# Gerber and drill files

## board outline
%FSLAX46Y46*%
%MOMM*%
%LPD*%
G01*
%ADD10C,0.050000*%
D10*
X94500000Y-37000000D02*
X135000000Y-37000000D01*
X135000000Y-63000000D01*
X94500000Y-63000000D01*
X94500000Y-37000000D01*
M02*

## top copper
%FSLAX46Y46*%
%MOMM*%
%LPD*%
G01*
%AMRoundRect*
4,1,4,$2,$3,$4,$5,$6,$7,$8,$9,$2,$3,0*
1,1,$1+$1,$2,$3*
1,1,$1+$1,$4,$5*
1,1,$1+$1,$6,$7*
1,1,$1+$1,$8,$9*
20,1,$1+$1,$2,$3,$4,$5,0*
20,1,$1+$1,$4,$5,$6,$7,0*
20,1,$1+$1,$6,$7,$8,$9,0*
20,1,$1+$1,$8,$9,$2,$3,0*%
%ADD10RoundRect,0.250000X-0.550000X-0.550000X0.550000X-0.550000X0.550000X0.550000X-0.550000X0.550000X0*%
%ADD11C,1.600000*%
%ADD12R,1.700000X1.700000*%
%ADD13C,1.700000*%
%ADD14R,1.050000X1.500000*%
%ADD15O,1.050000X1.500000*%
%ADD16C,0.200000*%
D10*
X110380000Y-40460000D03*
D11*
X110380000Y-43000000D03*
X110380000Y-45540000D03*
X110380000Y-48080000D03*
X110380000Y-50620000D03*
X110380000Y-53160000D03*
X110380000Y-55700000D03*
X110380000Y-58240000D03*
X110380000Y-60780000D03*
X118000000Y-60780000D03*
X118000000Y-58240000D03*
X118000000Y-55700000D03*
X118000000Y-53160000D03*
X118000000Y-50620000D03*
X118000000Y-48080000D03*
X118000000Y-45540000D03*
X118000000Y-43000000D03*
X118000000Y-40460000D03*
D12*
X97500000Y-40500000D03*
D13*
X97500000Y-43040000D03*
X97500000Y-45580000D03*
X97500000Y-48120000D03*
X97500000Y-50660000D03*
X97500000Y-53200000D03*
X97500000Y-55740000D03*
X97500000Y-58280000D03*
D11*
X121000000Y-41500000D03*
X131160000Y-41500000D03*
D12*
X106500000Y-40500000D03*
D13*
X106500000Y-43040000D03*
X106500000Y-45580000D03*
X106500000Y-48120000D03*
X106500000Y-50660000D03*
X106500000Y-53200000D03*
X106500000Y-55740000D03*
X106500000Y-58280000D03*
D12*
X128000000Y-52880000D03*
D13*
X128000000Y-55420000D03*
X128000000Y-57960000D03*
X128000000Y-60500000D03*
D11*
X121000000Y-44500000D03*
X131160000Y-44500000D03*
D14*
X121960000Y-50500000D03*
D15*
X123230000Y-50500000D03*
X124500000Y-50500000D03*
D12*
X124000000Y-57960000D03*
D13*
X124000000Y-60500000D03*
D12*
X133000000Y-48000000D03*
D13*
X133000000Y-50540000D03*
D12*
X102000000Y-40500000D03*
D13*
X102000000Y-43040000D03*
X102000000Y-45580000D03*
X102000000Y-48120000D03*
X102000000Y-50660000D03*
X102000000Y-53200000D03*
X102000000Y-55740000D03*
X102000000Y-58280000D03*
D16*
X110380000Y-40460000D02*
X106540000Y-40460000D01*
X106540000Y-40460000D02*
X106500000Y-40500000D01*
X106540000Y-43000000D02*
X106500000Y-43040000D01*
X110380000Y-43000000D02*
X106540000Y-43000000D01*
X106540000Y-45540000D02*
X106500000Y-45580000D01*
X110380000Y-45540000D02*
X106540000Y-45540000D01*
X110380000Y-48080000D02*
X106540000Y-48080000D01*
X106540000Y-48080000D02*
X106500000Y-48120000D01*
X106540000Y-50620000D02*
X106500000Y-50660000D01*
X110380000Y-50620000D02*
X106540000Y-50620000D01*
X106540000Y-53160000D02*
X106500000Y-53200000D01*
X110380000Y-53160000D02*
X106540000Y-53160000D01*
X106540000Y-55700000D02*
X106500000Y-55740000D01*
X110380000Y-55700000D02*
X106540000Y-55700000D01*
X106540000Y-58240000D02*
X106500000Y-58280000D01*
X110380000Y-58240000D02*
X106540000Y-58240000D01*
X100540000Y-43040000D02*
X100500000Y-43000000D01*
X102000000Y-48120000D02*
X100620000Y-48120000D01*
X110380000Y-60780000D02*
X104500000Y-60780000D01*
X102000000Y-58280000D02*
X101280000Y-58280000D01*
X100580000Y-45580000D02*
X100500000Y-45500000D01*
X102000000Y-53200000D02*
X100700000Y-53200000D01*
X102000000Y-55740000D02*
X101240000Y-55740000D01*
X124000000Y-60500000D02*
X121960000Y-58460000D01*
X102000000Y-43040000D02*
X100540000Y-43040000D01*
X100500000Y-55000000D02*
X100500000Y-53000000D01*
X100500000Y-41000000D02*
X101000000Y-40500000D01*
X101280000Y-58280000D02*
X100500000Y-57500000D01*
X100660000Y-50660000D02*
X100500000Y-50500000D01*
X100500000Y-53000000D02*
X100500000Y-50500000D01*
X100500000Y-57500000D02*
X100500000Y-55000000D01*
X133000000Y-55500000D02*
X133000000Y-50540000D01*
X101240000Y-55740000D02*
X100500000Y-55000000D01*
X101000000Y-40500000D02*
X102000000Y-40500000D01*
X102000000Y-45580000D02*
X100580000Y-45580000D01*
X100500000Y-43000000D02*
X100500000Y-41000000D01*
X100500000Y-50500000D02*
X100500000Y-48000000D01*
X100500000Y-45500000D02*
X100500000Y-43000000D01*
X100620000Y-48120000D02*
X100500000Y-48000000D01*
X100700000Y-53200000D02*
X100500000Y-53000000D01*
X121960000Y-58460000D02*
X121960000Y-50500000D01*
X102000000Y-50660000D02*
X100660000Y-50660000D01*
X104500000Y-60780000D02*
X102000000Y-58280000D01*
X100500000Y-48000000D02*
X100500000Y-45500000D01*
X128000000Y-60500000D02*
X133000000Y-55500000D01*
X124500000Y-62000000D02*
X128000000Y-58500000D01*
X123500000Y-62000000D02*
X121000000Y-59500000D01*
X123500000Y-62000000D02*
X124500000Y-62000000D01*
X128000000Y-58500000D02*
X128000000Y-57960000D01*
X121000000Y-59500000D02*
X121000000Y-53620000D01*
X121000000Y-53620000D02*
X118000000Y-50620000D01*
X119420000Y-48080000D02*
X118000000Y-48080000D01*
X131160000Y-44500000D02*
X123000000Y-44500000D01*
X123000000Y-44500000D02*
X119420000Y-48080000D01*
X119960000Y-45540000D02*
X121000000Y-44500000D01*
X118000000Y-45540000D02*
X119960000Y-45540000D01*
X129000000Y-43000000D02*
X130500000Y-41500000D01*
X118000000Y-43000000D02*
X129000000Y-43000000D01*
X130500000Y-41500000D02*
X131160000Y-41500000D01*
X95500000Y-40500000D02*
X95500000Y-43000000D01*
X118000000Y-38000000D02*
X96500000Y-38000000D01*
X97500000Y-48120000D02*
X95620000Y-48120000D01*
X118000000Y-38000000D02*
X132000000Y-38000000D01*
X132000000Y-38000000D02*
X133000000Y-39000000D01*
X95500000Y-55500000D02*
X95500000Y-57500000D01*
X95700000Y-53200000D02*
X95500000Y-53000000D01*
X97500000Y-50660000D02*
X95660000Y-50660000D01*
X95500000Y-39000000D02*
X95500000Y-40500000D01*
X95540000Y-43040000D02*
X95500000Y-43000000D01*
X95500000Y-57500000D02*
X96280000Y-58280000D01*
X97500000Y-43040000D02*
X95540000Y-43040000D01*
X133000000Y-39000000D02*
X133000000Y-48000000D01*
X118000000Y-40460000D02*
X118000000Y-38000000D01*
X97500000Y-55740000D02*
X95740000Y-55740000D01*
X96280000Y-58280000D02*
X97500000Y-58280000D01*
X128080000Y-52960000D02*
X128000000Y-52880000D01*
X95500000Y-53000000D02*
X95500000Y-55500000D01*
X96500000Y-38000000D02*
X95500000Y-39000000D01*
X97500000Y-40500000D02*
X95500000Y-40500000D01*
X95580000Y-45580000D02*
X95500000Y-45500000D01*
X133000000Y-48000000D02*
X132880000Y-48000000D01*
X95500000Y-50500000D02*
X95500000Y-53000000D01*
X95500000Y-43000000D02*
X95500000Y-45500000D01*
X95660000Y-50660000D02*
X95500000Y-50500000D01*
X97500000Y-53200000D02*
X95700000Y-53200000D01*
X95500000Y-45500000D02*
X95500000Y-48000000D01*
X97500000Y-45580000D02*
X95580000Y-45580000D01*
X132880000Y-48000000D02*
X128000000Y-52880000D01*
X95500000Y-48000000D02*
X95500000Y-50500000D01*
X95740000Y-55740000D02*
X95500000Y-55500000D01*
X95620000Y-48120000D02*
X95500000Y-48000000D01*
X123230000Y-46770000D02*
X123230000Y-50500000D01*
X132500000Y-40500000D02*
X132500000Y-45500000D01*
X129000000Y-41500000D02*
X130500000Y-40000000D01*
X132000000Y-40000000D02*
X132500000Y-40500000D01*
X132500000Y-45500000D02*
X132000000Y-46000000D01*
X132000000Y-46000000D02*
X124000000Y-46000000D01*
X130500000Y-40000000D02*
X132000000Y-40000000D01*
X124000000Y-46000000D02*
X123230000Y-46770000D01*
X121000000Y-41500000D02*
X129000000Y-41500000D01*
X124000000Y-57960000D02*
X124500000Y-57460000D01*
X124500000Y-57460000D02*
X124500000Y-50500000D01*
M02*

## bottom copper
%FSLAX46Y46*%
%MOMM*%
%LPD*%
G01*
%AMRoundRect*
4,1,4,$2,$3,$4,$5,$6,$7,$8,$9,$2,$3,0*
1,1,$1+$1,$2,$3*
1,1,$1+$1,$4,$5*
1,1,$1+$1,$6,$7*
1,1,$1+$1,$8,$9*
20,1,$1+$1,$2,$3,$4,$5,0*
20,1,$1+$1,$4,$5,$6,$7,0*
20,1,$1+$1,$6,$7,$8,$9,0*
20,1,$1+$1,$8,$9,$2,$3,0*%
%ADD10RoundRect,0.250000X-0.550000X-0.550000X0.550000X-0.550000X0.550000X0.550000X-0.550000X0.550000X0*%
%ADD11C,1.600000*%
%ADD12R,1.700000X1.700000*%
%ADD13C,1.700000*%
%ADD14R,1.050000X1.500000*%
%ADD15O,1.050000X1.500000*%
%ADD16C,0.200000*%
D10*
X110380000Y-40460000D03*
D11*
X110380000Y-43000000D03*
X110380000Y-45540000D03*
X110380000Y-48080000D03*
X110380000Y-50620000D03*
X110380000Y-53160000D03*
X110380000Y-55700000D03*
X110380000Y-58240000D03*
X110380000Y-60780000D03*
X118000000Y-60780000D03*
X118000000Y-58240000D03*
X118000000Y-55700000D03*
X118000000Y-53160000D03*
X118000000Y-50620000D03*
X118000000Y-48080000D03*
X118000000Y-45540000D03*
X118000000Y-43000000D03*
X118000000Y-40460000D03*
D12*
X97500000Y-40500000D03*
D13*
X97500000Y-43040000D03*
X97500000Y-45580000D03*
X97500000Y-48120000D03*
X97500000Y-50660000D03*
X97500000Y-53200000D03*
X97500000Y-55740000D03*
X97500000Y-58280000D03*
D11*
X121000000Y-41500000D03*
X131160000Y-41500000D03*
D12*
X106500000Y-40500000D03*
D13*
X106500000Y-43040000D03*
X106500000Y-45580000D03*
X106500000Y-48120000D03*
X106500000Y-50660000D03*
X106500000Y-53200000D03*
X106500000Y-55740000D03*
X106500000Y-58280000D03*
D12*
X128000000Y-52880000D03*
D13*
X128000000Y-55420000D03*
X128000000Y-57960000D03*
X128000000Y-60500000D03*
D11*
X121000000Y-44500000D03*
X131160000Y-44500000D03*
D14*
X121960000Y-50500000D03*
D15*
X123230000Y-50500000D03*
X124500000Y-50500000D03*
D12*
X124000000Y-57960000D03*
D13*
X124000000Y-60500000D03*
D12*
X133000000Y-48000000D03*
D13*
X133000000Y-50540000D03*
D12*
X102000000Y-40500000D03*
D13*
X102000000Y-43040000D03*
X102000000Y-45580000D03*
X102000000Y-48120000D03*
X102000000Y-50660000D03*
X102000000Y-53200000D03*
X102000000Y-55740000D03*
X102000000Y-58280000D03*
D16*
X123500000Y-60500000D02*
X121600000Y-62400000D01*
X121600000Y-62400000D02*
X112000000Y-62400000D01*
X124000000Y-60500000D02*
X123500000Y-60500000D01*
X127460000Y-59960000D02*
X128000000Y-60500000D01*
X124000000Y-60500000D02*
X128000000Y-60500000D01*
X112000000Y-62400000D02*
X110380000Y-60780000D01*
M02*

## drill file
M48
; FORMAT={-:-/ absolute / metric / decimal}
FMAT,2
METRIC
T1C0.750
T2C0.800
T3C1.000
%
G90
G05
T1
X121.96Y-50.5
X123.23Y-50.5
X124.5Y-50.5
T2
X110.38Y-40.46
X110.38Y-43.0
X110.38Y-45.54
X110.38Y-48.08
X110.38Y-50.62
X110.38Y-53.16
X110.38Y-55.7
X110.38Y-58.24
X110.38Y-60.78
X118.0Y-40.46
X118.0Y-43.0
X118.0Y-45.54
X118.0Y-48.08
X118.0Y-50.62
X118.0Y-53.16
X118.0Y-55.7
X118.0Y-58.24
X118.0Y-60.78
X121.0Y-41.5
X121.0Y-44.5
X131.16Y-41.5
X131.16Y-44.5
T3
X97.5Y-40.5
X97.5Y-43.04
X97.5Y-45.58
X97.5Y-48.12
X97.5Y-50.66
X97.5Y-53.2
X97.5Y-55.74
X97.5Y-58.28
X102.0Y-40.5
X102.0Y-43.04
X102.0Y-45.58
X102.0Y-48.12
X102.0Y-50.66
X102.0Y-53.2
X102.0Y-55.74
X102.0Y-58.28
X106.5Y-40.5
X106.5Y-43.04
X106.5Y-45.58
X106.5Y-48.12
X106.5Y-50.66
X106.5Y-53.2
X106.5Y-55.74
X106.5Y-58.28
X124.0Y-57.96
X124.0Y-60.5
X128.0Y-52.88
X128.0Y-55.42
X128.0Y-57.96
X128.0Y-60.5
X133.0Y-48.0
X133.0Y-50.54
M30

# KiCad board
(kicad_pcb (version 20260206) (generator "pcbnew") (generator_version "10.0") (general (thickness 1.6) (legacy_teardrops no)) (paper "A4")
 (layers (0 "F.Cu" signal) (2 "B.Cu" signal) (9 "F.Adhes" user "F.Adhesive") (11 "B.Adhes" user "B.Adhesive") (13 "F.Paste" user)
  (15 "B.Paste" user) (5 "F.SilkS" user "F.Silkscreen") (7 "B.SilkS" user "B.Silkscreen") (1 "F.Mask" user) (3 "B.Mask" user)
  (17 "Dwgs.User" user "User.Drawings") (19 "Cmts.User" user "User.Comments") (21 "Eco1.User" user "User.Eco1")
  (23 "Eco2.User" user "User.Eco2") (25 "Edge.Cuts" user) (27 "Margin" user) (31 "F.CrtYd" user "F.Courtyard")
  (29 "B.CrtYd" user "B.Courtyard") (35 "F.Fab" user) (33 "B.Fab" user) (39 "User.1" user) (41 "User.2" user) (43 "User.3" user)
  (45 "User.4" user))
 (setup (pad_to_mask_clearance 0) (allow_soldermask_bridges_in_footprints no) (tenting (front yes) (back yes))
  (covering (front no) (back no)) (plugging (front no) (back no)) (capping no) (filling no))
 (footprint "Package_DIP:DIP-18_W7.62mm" (layer "F.Cu") (at 110.38 40.46)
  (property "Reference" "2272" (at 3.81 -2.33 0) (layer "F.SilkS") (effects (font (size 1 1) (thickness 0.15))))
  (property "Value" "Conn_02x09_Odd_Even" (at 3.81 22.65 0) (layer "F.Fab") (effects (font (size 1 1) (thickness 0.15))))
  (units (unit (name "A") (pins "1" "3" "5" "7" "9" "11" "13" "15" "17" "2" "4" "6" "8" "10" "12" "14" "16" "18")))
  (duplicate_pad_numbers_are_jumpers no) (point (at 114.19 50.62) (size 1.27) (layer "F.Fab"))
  (pad "1" thru_hole roundrect (at 0 0) (size 1.6 1.6) (drill 0.8) (layers "*.Cu" "*.Mask") (remove_unused_layers no)
   (roundrect_rratio 0.15625) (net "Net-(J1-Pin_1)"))
  (pad "2" thru_hole circle (at 0 2.54) (size 1.6 1.6) (drill 0.8) (layers "*.Cu" "*.Mask") (remove_unused_layers no) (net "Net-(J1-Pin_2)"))
  (pad "3" thru_hole circle (at 0 5.08) (size 1.6 1.6) (drill 0.8) (layers "*.Cu" "*.Mask") (remove_unused_layers no) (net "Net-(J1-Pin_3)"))
  (pad "4" thru_hole circle (at 0 7.62) (size 1.6 1.6) (drill 0.8) (layers "*.Cu" "*.Mask") (remove_unused_layers no) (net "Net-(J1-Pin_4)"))
  (pad "5" thru_hole circle (at 0 10.16) (size 1.6 1.6) (drill 0.8) (layers "*.Cu" "*.Mask") (remove_unused_layers no)
   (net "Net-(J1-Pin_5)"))
  (pad "6" thru_hole circle (at 0 12.7) (size 1.6 1.6) (drill 0.8) (layers "*.Cu" "*.Mask") (remove_unused_layers no) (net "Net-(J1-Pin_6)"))
  (pad "7" thru_hole circle (at 0 15.24) (size 1.6 1.6) (drill 0.8) (layers "*.Cu" "*.Mask") (remove_unused_layers no)
   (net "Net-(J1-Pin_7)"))
  (pad "8" thru_hole circle (at 0 17.78) (size 1.6 1.6) (drill 0.8) (layers "*.Cu" "*.Mask") (remove_unused_layers no)
   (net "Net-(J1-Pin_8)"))
  (pad "9" thru_hole circle (at 0 20.32) (size 1.6 1.6) (drill 0.8) (layers "*.Cu" "*.Mask") (remove_unused_layers no) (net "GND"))
  (pad "10" thru_hole circle (at 7.62 20.32) (size 1.6 1.6) (drill 0.8) (layers "*.Cu" "*.Mask") (remove_unused_layers no)
   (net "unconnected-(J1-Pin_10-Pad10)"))
  (pad "11" thru_hole circle (at 7.62 17.78) (size 1.6 1.6) (drill 0.8) (layers "*.Cu" "*.Mask") (remove_unused_layers no)
   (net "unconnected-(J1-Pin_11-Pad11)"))
  (pad "12" thru_hole circle (at 7.62 15.24) (size 1.6 1.6) (drill 0.8) (layers "*.Cu" "*.Mask") (remove_unused_layers no)
   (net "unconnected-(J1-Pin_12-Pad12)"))
  (pad "13" thru_hole circle (at 7.62 12.7) (size 1.6 1.6) (drill 0.8) (layers "*.Cu" "*.Mask") (remove_unused_layers no)
   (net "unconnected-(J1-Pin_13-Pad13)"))
  (pad "14" thru_hole circle (at 7.62 10.16) (size 1.6 1.6) (drill 0.8) (layers "*.Cu" "*.Mask") (remove_unused_layers no)
   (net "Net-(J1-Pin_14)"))
  (pad "15" thru_hole circle (at 7.62 7.62) (size 1.6 1.6) (drill 0.8) (layers "*.Cu" "*.Mask") (remove_unused_layers no)
   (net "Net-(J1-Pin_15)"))
  (pad "16" thru_hole circle (at 7.62 5.08) (size 1.6 1.6) (drill 0.8) (layers "*.Cu" "*.Mask") (remove_unused_layers no)
   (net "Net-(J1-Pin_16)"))
  (pad "17" thru_hole circle (at 7.62 2.54) (size 1.6 1.6) (drill 0.8) (layers "*.Cu" "*.Mask") (remove_unused_layers no)
   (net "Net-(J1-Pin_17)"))
  (pad "18" thru_hole circle (at 7.62 0) (size 1.6 1.6) (drill 0.8) (layers "*.Cu" "*.Mask") (remove_unused_layers no) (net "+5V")))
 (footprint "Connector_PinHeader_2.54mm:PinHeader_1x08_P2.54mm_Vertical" (layer "F.Cu") (at 97.5 40.5)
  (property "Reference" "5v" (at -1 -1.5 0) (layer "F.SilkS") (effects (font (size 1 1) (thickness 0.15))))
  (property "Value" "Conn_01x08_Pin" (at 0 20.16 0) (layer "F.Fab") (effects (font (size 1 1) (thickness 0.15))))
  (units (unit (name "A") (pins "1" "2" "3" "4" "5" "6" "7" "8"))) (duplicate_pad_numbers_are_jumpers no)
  (pad "1" thru_hole rect (at 0 0) (size 1.7 1.7) (drill 1) (layers "*.Cu" "*.Mask") (remove_unused_layers no) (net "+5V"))
  (pad "2" thru_hole circle (at 0 2.54) (size 1.7 1.7) (drill 1) (layers "*.Cu" "*.Mask") (remove_unused_layers no) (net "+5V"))
  (pad "3" thru_hole circle (at 0 5.08) (size 1.7 1.7) (drill 1) (layers "*.Cu" "*.Mask") (remove_unused_layers no) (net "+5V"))
  (pad "4" thru_hole circle (at 0 7.62) (size 1.7 1.7) (drill 1) (layers "*.Cu" "*.Mask") (remove_unused_layers no) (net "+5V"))
  (pad "5" thru_hole circle (at 0 10.16) (size 1.7 1.7) (drill 1) (layers "*.Cu" "*.Mask") (remove_unused_layers no) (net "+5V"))
  (pad "6" thru_hole circle (at 0 12.7) (size 1.7 1.7) (drill 1) (layers "*.Cu" "*.Mask") (remove_unused_layers no) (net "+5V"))
  (pad "7" thru_hole circle (at 0 15.24) (size 1.7 1.7) (drill 1) (layers "*.Cu" "*.Mask") (remove_unused_layers no) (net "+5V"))
  (pad "8" thru_hole circle (at 0 17.78) (size 1.7 1.7) (drill 1) (layers "*.Cu" "*.Mask") (remove_unused_layers no) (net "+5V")))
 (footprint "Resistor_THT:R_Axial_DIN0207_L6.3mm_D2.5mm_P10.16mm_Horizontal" (layer "F.Cu") (at 121 41.5)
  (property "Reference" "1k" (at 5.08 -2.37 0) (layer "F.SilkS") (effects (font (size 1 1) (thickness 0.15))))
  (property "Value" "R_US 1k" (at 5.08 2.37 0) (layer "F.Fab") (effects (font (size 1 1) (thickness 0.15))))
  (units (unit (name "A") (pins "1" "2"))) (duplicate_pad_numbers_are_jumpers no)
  (pad "1" thru_hole circle (at 0 0) (size 1.6 1.6) (drill 0.8) (layers "*.Cu" "*.Mask") (remove_unused_layers no) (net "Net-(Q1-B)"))
  (pad "2" thru_hole circle (at 10.16 0) (size 1.6 1.6) (drill 0.8) (layers "*.Cu" "*.Mask") (remove_unused_layers no)
   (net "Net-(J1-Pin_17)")))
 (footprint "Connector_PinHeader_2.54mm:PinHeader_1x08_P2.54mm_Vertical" (layer "F.Cu") (at 106.5 40.5)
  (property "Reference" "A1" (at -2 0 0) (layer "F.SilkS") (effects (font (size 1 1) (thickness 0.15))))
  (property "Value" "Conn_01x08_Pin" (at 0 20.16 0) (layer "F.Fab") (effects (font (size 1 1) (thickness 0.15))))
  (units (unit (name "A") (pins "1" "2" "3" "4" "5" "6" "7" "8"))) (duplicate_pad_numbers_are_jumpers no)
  (pad "1" thru_hole rect (at 0 0) (size 1.7 1.7) (drill 1) (layers "*.Cu" "*.Mask") (remove_unused_layers no) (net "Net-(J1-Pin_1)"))
  (pad "2" thru_hole circle (at 0 2.54) (size 1.7 1.7) (drill 1) (layers "*.Cu" "*.Mask") (remove_unused_layers no) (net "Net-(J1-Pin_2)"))
  (pad "3" thru_hole circle (at 0 5.08) (size 1.7 1.7) (drill 1) (layers "*.Cu" "*.Mask") (remove_unused_layers no) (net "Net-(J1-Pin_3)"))
  (pad "4" thru_hole circle (at 0 7.62) (size 1.7 1.7) (drill 1) (layers "*.Cu" "*.Mask") (remove_unused_layers no) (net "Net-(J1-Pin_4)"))
  (pad "5" thru_hole circle (at 0 10.16) (size 1.7 1.7) (drill 1) (layers "*.Cu" "*.Mask") (remove_unused_layers no) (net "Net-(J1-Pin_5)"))
  (pad "6" thru_hole circle (at 0 12.7) (size 1.7 1.7) (drill 1) (layers "*.Cu" "*.Mask") (remove_unused_layers no) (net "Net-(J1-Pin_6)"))
  (pad "7" thru_hole circle (at 0 15.24) (size 1.7 1.7) (drill 1) (layers "*.Cu" "*.Mask") (remove_unused_layers no) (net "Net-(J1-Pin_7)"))
  (pad "8" thru_hole circle (at 0 17.78) (size 1.7 1.7) (drill 1) (layers "*.Cu" "*.Mask") (remove_unused_layers no) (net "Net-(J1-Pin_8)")))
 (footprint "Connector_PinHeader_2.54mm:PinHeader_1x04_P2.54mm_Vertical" (layer "F.Cu") (at 128 52.88)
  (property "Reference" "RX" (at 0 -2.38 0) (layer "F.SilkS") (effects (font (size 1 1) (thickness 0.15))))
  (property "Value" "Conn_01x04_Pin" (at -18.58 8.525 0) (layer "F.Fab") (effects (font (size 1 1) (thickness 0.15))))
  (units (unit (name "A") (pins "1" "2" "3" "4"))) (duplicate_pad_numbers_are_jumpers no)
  (pad "1" thru_hole rect (at 0 0) (size 1.7 1.7) (drill 1) (layers "*.Cu" "*.Mask") (remove_unused_layers no) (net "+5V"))
  (pad "2" thru_hole circle (at 0 2.54) (size 1.7 1.7) (drill 1) (layers "*.Cu" "*.Mask") (remove_unused_layers no)
   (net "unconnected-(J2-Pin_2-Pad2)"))
  (pad "3" thru_hole circle (at 0 5.08) (size 1.7 1.7) (drill 1) (layers "*.Cu" "*.Mask") (remove_unused_layers no) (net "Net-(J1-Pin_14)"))
  (pad "4" thru_hole circle (at 0 7.62) (size 1.7 1.7) (drill 1) (layers "*.Cu" "*.Mask") (remove_unused_layers no) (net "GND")))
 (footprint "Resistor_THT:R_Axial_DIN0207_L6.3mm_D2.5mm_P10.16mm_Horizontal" (layer "F.Cu") (at 121 44.5)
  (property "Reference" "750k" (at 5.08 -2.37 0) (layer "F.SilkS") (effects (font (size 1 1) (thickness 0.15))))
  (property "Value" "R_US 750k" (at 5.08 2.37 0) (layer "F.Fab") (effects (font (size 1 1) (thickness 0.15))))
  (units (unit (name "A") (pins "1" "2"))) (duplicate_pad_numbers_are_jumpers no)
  (pad "1" thru_hole circle (at 0 0) (size 1.6 1.6) (drill 0.8) (layers "*.Cu" "*.Mask") (remove_unused_layers no) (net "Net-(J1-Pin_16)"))
  (pad "2" thru_hole circle (at 10.16 0) (size 1.6 1.6) (drill 0.8) (layers "*.Cu" "*.Mask") (remove_unused_layers no)
   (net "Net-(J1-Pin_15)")))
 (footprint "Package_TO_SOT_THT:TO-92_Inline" (layer "F.Cu") (at 121.96 50.5)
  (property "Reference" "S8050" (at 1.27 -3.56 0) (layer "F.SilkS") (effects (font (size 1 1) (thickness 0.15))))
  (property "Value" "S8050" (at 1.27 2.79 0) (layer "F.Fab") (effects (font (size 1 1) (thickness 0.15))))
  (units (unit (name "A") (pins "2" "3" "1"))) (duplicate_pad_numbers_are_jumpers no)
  (pad "1" thru_hole rect (at 0 0) (size 1.05 1.5) (drill 0.75) (layers "*.Cu" "*.Mask") (remove_unused_layers no) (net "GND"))
  (pad "2" thru_hole oval (at 1.27 0) (size 1.05 1.5) (drill 0.75) (layers "*.Cu" "*.Mask") (remove_unused_layers no) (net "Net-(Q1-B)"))
  (pad "3" thru_hole oval (at 2.54 0) (size 1.05 1.5) (drill 0.75) (layers "*.Cu" "*.Mask") (remove_unused_layers no) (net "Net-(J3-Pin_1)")))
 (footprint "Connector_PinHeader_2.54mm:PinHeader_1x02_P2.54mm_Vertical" (layer "F.Cu") (at 124 57.96)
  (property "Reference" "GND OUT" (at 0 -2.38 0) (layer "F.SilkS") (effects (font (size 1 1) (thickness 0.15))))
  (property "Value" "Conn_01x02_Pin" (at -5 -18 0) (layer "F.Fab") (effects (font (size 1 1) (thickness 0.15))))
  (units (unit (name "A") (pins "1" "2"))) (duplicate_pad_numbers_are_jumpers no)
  (pad "1" thru_hole rect (at 0 0) (size 1.7 1.7) (drill 1) (layers "*.Cu" "*.Mask") (remove_unused_layers no) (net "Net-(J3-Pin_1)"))
  (pad "2" thru_hole circle (at 0 2.54) (size 1.7 1.7) (drill 1) (layers "*.Cu" "*.Mask") (remove_unused_layers no) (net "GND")))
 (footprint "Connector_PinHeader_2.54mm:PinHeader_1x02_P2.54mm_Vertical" (layer "F.Cu") (at 133 48)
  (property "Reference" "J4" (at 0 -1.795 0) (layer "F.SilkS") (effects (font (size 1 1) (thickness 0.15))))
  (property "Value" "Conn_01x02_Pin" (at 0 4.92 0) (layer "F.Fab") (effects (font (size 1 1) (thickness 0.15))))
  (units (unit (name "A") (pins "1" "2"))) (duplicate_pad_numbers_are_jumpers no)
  (pad "1" thru_hole rect (at 0 0) (size 1.7 1.7) (drill 1) (layers "*.Cu" "*.Mask") (remove_unused_layers no) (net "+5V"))
  (pad "2" thru_hole circle (at 0 2.54) (size 1.7 1.7) (drill 1) (layers "*.Cu" "*.Mask") (remove_unused_layers no) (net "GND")))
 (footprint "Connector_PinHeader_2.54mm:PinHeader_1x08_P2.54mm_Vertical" (layer "F.Cu") (at 102 40.5)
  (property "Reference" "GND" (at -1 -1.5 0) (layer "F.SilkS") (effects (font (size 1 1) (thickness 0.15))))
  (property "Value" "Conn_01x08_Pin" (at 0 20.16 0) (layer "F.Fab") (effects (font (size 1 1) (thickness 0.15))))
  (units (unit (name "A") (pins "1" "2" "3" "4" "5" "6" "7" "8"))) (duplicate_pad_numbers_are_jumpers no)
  (pad "1" thru_hole rect (at 0 0) (size 1.7 1.7) (drill 1) (layers "*.Cu" "*.Mask") (remove_unused_layers no) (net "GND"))
  (pad "2" thru_hole circle (at 0 2.54) (size 1.7 1.7) (drill 1) (layers "*.Cu" "*.Mask") (remove_unused_layers no) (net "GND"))
  (pad "3" thru_hole circle (at 0 5.08) (size 1.7 1.7) (drill 1) (layers "*.Cu" "*.Mask") (remove_unused_layers no) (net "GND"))
  (pad "4" thru_hole circle (at 0 7.62) (size 1.7 1.7) (drill 1) (layers "*.Cu" "*.Mask") (remove_unused_layers no) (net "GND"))
  (pad "5" thru_hole circle (at 0 10.16) (size 1.7 1.7) (drill 1) (layers "*.Cu" "*.Mask") (remove_unused_layers no) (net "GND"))
  (pad "6" thru_hole circle (at 0 12.7) (size 1.7 1.7) (drill 1) (layers "*.Cu" "*.Mask") (remove_unused_layers no) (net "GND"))
  (pad "7" thru_hole circle (at 0 15.24) (size 1.7 1.7) (drill 1) (layers "*.Cu" "*.Mask") (remove_unused_layers no) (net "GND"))
  (pad "8" thru_hole circle (at 0 17.78) (size 1.7 1.7) (drill 1) (layers "*.Cu" "*.Mask") (remove_unused_layers no) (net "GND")))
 (gr_rect (start 94.5 37) (end 135 63) (stroke (width 0.05) (type default)) (fill no) (layer "Edge.Cuts"))
 (segment (start 110.38 40.46) (end 106.54 40.46) (width 0.2) (layer "F.Cu") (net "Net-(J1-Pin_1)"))
 (segment (start 106.54 40.46) (end 106.5 40.5) (width 0.2) (layer "F.Cu") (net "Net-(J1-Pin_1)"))
 (segment (start 106.54 43) (end 106.5 43.04) (width 0.2) (layer "F.Cu") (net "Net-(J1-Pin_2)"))
 (segment (start 110.38 43) (end 106.54 43) (width 0.2) (layer "F.Cu") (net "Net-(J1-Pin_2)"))
 (segment (start 106.54 45.54) (end 106.5 45.58) (width 0.2) (layer "F.Cu") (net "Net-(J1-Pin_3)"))
 (segment (start 110.38 45.54) (end 106.54 45.54) (width 0.2) (layer "F.Cu") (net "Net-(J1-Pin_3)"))
 (segment (start 110.38 48.08) (end 106.54 48.08) (width 0.2) (layer "F.Cu") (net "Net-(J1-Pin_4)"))
 (segment (start 106.54 48.08) (end 106.5 48.12) (width 0.2) (layer "F.Cu") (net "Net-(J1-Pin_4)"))
 (segment (start 106.54 50.62) (end 106.5 50.66) (width 0.2) (layer "F.Cu") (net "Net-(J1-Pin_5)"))
 (segment (start 110.38 50.62) (end 106.54 50.62) (width 0.2) (layer "F.Cu") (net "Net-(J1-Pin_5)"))
 (segment (start 106.54 53.16) (end 106.5 53.2) (width 0.2) (layer "F.Cu") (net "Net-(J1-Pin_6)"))
 (segment (start 110.38 53.16) (end 106.54 53.16) (width 0.2) (layer "F.Cu") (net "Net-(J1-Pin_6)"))
 (segment (start 106.54 55.7) (end 106.5 55.74) (width 0.2) (layer "F.Cu") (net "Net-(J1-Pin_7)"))
 (segment (start 110.38 55.7) (end 106.54 55.7) (width 0.2) (layer "F.Cu") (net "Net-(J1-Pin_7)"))
 (segment (start 106.54 58.24) (end 106.5 58.28) (width 0.2) (layer "F.Cu") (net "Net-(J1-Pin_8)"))
 (segment (start 110.38 58.24) (end 106.54 58.24) (width 0.2) (layer "F.Cu") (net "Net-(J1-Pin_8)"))
 (segment (start 100.54 43.04) (end 100.5 43) (width 0.2) (layer "F.Cu") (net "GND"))
 (segment (start 102 48.12) (end 100.62 48.12) (width 0.2) (layer "F.Cu") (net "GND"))
 (segment (start 110.38 60.78) (end 104.5 60.78) (width 0.2) (layer "F.Cu") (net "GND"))
 (segment (start 102 58.28) (end 101.28 58.28) (width 0.2) (layer "F.Cu") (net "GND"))
 (segment (start 100.58 45.58) (end 100.5 45.5) (width 0.2) (layer "F.Cu") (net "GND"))
 (segment (start 102 53.2) (end 100.7 53.2) (width 0.2) (layer "F.Cu") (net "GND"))
 (segment (start 102 55.74) (end 101.24 55.74) (width 0.2) (layer "F.Cu") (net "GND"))
 (segment (start 124 60.5) (end 121.96 58.46) (width 0.2) (layer "F.Cu") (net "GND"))
 (segment (start 102 43.04) (end 100.54 43.04) (width 0.2) (layer "F.Cu") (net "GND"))
 (segment (start 100.5 55) (end 100.5 53) (width 0.2) (layer "F.Cu") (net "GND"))
 (segment (start 100.5 41) (end 101 40.5) (width 0.2) (layer "F.Cu") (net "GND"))
 (segment (start 101.28 58.28) (end 100.5 57.5) (width 0.2) (layer "F.Cu") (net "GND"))
 (segment (start 100.66 50.66) (end 100.5 50.5) (width 0.2) (layer "F.Cu") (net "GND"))
 (segment (start 100.5 53) (end 100.5 50.5) (width 0.2) (layer "F.Cu") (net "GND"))
 (segment (start 100.5 57.5) (end 100.5 55) (width 0.2) (layer "F.Cu") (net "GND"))
 (segment (start 133 55.5) (end 133 50.54) (width 0.2) (layer "F.Cu") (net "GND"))
 (segment (start 101.24 55.74) (end 100.5 55) (width 0.2) (layer "F.Cu") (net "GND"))
 (segment (start 101 40.5) (end 102 40.5) (width 0.2) (layer "F.Cu") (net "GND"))
 (segment (start 102 45.58) (end 100.58 45.58) (width 0.2) (layer "F.Cu") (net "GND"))
 (segment (start 100.5 43) (end 100.5 41) (width 0.2) (layer "F.Cu") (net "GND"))
 (segment (start 100.5 50.5) (end 100.5 48) (width 0.2) (layer "F.Cu") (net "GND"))
 (segment (start 100.5 45.5) (end 100.5 43) (width 0.2) (layer "F.Cu") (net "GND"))
 (segment (start 100.62 48.12) (end 100.5 48) (width 0.2) (layer "F.Cu") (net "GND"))
 (segment (start 100.7 53.2) (end 100.5 53) (width 0.2) (layer "F.Cu") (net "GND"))
 (segment (start 121.96 58.46) (end 121.96 50.5) (width 0.2) (layer "F.Cu") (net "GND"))
 (segment (start 102 50.66) (end 100.66 50.66) (width 0.2) (layer "F.Cu") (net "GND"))
 (segment (start 104.5 60.78) (end 102 58.28) (width 0.2) (layer "F.Cu") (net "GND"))
 (segment (start 100.5 48) (end 100.5 45.5) (width 0.2) (layer "F.Cu") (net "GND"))
 (segment (start 128 60.5) (end 133 55.5) (width 0.2) (layer "F.Cu") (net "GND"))
 (segment (start 123.5 60.5) (end 121.6 62.4) (width 0.2) (layer "B.Cu") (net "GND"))
 (segment (start 121.6 62.4) (end 112 62.4) (width 0.2) (layer "B.Cu") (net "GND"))
 (segment (start 124 60.5) (end 123.5 60.5) (width 0.2) (layer "B.Cu") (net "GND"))
 (segment (start 127.46 59.96) (end 128 60.5) (width 0.2) (layer "B.Cu") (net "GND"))
 (segment (start 124 60.5) (end 128 60.5) (width 0.2) (layer "B.Cu") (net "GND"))
 (segment (start 112 62.4) (end 110.38 60.78) (width 0.2) (layer "B.Cu") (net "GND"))
 (segment (start 124.5 62) (end 128 58.5) (width 0.2) (layer "F.Cu") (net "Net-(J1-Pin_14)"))
 (segment (start 123.5 62) (end 121 59.5) (width 0.2) (layer "F.Cu") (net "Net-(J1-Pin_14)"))
 (segment (start 123.5 62) (end 124.5 62) (width 0.2) (layer "F.Cu") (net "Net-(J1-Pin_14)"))
 (segment (start 128 58.5) (end 128 57.96) (width 0.2) (layer "F.Cu") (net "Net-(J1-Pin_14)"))
 (segment (start 121 59.5) (end 121 53.62) (width 0.2) (layer "F.Cu") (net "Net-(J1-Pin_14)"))
 (segment (start 121 53.62) (end 118 50.62) (width 0.2) (layer "F.Cu") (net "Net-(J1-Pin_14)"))
 (segment (start 119.42 48.08) (end 118 48.08) (width 0.2) (layer "F.Cu") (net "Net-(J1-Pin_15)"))
 (segment (start 131.16 44.5) (end 123 44.5) (width 0.2) (layer "F.Cu") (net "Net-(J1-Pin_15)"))
 (segment (start 123 44.5) (end 119.42 48.08) (width 0.2) (layer "F.Cu") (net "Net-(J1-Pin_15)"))
 (segment (start 119.96 45.54) (end 121 44.5) (width 0.2) (layer "F.Cu") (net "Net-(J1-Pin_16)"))
 (segment (start 118 45.54) (end 119.96 45.54) (width 0.2) (layer "F.Cu") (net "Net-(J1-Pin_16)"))
 (segment (start 129 43) (end 130.5 41.5) (width 0.2) (layer "F.Cu") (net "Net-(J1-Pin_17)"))
 (segment (start 118 43) (end 129 43) (width 0.2) (layer "F.Cu") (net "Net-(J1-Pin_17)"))
 (segment (start 130.5 41.5) (end 131.16 41.5) (width 0.2) (layer "F.Cu") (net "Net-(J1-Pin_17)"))
 (segment (start 95.5 40.5) (end 95.5 43) (width 0.2) (layer "F.Cu") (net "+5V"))
 (segment (start 118 38) (end 96.5 38) (width 0.2) (layer "F.Cu") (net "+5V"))
 (segment (start 97.5 48.12) (end 95.62 48.12) (width 0.2) (layer "F.Cu") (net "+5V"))
 (segment (start 118 38) (end 132 38) (width 0.2) (layer "F.Cu") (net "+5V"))
 (segment (start 132 38) (end 133 39) (width 0.2) (layer "F.Cu") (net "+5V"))
 (segment (start 95.5 55.5) (end 95.5 57.5) (width 0.2) (layer "F.Cu") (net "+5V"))
 (segment (start 95.7 53.2) (end 95.5 53) (width 0.2) (layer "F.Cu") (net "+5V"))
 (segment (start 97.5 50.66) (end 95.66 50.66) (width 0.2) (layer "F.Cu") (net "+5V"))
 (segment (start 95.5 39) (end 95.5 40.5) (width 0.2) (layer "F.Cu") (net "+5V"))
 (segment (start 95.54 43.04) (end 95.5 43) (width 0.2) (layer "F.Cu") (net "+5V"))
 (segment (start 95.5 57.5) (end 96.28 58.28) (width 0.2) (layer "F.Cu") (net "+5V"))
 (segment (start 97.5 43.04) (end 95.54 43.04) (width 0.2) (layer "F.Cu") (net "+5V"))
 (segment (start 133 39) (end 133 48) (width 0.2) (layer "F.Cu") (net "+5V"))
 (segment (start 118 40.46) (end 118 38) (width 0.2) (layer "F.Cu") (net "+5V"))
 (segment (start 97.5 55.74) (end 95.74 55.74) (width 0.2) (layer "F.Cu") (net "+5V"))
 (segment (start 96.28 58.28) (end 97.5 58.28) (width 0.2) (layer "F.Cu") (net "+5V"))
 (segment (start 128.08 52.96) (end 128 52.88) (width 0.2) (layer "F.Cu") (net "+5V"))
 (segment (start 95.5 53) (end 95.5 55.5) (width 0.2) (layer "F.Cu") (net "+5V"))
 (segment (start 96.5 38) (end 95.5 39) (width 0.2) (layer "F.Cu") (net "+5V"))
 (segment (start 97.5 40.5) (end 95.5 40.5) (width 0.2) (layer "F.Cu") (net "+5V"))
 (segment (start 95.58 45.58) (end 95.5 45.5) (width 0.2) (layer "F.Cu") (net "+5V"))
 (segment (start 133 48) (end 132.88 48) (width 0.2) (layer "F.Cu") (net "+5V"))
 (segment (start 95.5 50.5) (end 95.5 53) (width 0.2) (layer "F.Cu") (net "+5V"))
 (segment (start 95.5 43) (end 95.5 45.5) (width 0.2) (layer "F.Cu") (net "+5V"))
 (segment (start 95.66 50.66) (end 95.5 50.5) (width 0.2) (layer "F.Cu") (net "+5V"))
 (segment (start 97.5 53.2) (end 95.7 53.2) (width 0.2) (layer "F.Cu") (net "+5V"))
 (segment (start 95.5 45.5) (end 95.5 48) (width 0.2) (layer "F.Cu") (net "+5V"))
 (segment (start 97.5 45.58) (end 95.58 45.58) (width 0.2) (layer "F.Cu") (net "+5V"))
 (segment (start 132.88 48) (end 128 52.88) (width 0.2) (layer "F.Cu") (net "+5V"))
 (segment (start 95.5 48) (end 95.5 50.5) (width 0.2) (layer "F.Cu") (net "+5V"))
 (segment (start 95.74 55.74) (end 95.5 55.5) (width 0.2) (layer "F.Cu") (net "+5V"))
 (segment (start 95.62 48.12) (end 95.5 48) (width 0.2) (layer "F.Cu") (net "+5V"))
 (segment (start 123.23 46.77) (end 123.23 50.5) (width 0.2) (layer "F.Cu") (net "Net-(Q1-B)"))
 (segment (start 132.5 40.5) (end 132.5 45.5) (width 0.2) (layer "F.Cu") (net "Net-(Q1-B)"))
 (segment (start 129 41.5) (end 130.5 40) (width 0.2) (layer "F.Cu") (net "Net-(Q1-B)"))
 (segment (start 132 40) (end 132.5 40.5) (width 0.2) (layer "F.Cu") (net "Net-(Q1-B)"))
 (segment (start 132.5 45.5) (end 132 46) (width 0.2) (layer "F.Cu") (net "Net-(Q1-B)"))
 (segment (start 132 46) (end 124 46) (width 0.2) (layer "F.Cu") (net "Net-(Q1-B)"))
 (segment (start 130.5 40) (end 132 40) (width 0.2) (layer "F.Cu") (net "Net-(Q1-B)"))
 (segment (start 124 46) (end 123.23 46.77) (width 0.2) (layer "F.Cu") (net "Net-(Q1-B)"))
 (segment (start 121 41.5) (end 129 41.5) (width 0.2) (layer "F.Cu") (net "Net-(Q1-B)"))
 (segment (start 124 57.96) (end 124.5 57.46) (width 0.2) (layer "F.Cu") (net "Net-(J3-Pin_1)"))
 (segment (start 124.5 57.46) (end 124.5 50.5) (width 0.2) (layer "F.Cu") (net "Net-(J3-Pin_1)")))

